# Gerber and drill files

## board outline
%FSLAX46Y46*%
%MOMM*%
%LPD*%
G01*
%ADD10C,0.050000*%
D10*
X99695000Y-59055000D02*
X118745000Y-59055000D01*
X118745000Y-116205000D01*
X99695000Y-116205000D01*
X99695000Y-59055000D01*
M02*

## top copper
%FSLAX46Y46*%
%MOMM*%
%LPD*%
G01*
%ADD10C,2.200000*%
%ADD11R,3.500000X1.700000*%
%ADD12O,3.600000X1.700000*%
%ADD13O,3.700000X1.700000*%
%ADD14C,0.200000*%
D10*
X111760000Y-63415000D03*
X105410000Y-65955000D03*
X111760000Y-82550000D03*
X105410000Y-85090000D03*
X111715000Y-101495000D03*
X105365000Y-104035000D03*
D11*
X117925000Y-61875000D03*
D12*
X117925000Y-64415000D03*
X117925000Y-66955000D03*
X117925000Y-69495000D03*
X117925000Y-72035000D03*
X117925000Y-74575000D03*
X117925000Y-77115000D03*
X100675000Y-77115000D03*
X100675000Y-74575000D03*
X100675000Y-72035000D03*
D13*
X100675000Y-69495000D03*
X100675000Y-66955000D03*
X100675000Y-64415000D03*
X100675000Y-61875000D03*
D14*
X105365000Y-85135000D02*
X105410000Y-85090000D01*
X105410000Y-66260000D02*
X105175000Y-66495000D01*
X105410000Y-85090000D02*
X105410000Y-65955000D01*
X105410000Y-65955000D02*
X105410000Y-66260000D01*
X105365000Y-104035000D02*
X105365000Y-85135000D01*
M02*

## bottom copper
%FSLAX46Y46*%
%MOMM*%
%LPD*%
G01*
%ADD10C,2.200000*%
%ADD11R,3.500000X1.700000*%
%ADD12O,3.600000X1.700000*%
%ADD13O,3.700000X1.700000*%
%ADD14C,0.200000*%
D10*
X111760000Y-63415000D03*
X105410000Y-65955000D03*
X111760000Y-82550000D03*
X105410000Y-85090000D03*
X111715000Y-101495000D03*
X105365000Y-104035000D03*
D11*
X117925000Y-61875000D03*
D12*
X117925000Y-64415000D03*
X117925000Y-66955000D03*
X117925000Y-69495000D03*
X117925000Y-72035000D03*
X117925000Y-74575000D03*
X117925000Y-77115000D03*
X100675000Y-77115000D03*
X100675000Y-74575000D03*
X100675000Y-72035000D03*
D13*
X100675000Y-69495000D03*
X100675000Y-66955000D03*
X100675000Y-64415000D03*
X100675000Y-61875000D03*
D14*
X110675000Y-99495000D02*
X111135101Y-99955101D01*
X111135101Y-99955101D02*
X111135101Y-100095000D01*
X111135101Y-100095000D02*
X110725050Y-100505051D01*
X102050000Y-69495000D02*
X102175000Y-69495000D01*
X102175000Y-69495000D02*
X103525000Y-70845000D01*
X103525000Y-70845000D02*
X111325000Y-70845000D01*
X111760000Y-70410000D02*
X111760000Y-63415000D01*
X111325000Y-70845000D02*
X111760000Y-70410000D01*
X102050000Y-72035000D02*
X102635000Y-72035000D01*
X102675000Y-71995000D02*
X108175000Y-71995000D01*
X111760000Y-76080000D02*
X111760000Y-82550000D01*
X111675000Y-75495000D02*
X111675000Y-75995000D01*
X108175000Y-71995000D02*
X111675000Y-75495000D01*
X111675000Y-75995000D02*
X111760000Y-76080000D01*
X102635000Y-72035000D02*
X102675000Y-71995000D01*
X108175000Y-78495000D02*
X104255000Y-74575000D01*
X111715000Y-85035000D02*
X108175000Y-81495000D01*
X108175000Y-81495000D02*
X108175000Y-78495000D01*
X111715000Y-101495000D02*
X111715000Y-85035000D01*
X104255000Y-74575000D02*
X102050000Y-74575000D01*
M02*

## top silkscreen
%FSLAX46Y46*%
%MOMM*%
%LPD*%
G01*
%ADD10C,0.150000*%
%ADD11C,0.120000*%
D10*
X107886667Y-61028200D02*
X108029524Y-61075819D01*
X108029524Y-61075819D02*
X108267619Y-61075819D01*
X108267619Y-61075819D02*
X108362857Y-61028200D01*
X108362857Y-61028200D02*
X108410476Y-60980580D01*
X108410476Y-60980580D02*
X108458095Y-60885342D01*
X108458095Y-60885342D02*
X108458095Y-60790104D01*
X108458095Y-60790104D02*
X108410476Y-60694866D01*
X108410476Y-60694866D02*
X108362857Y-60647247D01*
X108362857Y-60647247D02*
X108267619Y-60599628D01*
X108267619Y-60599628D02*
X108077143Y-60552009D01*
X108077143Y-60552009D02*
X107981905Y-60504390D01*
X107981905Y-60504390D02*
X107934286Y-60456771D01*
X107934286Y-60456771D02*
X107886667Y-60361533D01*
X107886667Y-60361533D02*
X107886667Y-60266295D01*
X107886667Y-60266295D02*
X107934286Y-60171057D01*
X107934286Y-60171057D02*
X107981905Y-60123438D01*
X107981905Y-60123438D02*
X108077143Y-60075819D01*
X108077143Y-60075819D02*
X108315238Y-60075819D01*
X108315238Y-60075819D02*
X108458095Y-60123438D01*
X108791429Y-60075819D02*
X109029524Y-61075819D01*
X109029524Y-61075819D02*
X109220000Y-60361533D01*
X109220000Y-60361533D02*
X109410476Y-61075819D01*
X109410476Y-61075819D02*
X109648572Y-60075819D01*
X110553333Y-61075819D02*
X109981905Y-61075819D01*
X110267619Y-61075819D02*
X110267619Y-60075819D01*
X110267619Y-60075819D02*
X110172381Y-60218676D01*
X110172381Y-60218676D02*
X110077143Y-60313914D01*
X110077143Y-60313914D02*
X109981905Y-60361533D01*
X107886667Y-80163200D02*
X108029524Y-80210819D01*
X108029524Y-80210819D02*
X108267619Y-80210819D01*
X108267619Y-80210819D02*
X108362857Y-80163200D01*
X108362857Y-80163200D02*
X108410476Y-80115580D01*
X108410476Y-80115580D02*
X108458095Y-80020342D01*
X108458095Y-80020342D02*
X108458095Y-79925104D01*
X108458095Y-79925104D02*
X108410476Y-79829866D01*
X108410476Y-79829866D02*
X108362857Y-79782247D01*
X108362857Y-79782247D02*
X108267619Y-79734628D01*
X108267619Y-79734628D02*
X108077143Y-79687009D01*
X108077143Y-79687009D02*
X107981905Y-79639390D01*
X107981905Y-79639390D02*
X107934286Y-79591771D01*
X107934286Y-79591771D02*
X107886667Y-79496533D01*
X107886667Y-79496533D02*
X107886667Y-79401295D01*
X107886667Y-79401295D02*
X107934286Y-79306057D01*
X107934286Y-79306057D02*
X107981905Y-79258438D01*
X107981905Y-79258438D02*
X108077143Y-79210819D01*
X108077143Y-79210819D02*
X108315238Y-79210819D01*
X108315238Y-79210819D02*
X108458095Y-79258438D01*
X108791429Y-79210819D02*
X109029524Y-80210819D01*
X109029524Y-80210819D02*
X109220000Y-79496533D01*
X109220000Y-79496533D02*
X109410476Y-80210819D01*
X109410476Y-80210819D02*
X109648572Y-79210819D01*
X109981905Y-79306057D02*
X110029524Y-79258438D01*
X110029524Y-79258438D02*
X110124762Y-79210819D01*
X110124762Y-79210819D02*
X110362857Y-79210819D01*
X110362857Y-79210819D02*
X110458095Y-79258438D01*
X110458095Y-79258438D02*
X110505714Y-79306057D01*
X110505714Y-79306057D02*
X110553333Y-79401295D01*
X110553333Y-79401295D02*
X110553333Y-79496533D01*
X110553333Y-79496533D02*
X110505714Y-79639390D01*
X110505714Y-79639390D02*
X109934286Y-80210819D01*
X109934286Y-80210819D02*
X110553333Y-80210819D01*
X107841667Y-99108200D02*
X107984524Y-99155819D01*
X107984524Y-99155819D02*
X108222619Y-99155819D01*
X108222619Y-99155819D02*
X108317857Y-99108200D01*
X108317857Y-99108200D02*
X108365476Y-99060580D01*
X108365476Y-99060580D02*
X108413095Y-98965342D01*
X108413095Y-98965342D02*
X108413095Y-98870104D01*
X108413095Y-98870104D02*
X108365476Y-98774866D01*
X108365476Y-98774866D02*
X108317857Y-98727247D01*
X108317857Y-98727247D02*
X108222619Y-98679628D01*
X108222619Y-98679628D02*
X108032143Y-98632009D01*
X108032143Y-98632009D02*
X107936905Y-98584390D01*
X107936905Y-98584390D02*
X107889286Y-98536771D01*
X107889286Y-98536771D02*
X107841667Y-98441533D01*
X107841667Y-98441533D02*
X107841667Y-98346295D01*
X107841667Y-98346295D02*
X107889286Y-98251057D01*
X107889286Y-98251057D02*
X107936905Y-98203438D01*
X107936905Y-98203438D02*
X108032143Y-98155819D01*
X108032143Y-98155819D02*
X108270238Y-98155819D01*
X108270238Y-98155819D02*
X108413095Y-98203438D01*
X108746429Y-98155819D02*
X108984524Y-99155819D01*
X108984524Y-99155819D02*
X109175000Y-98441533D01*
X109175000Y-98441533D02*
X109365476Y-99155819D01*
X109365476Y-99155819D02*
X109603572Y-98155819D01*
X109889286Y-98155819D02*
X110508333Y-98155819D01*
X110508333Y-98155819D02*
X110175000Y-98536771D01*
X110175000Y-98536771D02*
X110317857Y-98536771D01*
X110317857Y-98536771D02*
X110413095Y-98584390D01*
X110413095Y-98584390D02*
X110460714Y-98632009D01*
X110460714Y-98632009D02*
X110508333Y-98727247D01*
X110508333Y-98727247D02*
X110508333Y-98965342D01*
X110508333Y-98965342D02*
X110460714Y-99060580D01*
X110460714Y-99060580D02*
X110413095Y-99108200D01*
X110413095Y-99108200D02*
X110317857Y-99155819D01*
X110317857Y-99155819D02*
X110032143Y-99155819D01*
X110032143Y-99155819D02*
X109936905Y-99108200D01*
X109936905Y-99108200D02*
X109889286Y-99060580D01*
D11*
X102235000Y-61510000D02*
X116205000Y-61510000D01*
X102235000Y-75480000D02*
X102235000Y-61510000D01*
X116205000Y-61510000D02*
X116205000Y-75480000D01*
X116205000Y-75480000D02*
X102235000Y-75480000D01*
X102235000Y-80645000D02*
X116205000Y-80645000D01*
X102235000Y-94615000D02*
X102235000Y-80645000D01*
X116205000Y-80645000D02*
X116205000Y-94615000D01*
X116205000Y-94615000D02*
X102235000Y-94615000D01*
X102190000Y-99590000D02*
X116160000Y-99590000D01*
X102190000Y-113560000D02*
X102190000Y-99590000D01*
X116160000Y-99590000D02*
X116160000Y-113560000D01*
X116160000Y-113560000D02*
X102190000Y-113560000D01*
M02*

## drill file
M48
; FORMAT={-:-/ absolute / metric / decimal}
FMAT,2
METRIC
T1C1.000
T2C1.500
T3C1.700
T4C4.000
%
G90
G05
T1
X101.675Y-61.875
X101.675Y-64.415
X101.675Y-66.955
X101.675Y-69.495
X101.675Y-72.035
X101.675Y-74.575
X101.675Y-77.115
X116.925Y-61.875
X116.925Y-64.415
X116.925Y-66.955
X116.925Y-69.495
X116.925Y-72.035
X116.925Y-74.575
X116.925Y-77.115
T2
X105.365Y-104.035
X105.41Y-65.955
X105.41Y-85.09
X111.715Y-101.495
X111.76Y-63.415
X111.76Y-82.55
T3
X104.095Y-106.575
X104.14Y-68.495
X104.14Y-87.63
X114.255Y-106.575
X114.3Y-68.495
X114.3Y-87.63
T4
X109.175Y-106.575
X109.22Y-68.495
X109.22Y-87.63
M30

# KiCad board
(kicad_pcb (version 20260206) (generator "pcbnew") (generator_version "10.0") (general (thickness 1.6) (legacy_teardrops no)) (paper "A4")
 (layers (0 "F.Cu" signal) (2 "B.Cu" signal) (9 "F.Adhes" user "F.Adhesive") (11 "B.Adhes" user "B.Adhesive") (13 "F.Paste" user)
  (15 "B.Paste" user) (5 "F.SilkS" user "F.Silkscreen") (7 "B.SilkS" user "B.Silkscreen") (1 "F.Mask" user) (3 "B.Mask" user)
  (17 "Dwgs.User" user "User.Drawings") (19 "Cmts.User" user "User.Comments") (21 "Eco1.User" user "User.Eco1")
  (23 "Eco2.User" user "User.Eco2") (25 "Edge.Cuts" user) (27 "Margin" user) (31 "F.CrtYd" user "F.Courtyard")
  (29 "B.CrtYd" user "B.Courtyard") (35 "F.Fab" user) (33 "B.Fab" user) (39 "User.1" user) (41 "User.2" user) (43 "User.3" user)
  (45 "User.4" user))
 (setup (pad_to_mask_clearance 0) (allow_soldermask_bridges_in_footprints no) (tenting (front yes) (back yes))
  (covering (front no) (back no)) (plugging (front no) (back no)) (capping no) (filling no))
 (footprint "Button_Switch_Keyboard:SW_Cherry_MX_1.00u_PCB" (layer "F.Cu") (at 111.76 63.415)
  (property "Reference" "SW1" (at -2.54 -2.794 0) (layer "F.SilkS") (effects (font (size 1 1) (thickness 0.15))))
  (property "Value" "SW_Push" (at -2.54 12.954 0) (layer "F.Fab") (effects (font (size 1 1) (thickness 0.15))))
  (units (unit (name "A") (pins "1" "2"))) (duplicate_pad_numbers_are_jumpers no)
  (fp_line (start -9.525 -1.905) (end 4.445 -1.905) (stroke (width 0.12) (type solid)) (layer "F.SilkS"))
  (fp_line (start -9.525 12.065) (end -9.525 -1.905) (stroke (width 0.12) (type solid)) (layer "F.SilkS"))
  (fp_line (start 4.445 -1.905) (end 4.445 12.065) (stroke (width 0.12) (type solid)) (layer "F.SilkS"))
  (fp_line (start 4.445 12.065) (end -9.525 12.065) (stroke (width 0.12) (type solid)) (layer "F.SilkS"))
  (pad "" np_thru_hole circle (at -7.62 5.08) (size 1.7 1.7) (drill 1.7) (layers "*.Cu" "*.Mask"))
  (pad "" np_thru_hole circle (at -2.54 5.08) (size 4 4) (drill 4) (layers "*.Cu" "*.Mask"))
  (pad "" np_thru_hole circle (at 2.54 5.08) (size 1.7 1.7) (drill 1.7) (layers "*.Cu" "*.Mask"))
  (pad "1" thru_hole circle (at 0 0) (size 2.2 2.2) (drill 1.5) (layers "*.Cu" "*.Mask") (remove_unused_layers no)
   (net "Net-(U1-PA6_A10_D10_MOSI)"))
  (pad "2" thru_hole circle (at -6.35 2.54) (size 2.2 2.2) (drill 1.5) (layers "*.Cu" "*.Mask") (remove_unused_layers no) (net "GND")))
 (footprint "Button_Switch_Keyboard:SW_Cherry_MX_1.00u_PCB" (layer "F.Cu") (at 111.76 82.55)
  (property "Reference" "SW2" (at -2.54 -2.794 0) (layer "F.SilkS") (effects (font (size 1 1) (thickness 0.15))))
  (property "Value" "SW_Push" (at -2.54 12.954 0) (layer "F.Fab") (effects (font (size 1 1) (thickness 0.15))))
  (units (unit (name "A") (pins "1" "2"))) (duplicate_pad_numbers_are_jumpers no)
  (fp_line (start -9.525 -1.905) (end 4.445 -1.905) (stroke (width 0.12) (type solid)) (layer "F.SilkS"))
  (fp_line (start -9.525 12.065) (end -9.525 -1.905) (stroke (width 0.12) (type solid)) (layer "F.SilkS"))
  (fp_line (start 4.445 -1.905) (end 4.445 12.065) (stroke (width 0.12) (type solid)) (layer "F.SilkS"))
  (fp_line (start 4.445 12.065) (end -9.525 12.065) (stroke (width 0.12) (type solid)) (layer "F.SilkS"))
  (pad "" np_thru_hole circle (at -7.62 5.08) (size 1.7 1.7) (drill 1.7) (layers "*.Cu" "*.Mask"))
  (pad "" np_thru_hole circle (at -2.54 5.08) (size 4 4) (drill 4) (layers "*.Cu" "*.Mask"))
  (pad "" np_thru_hole circle (at 2.54 5.08) (size 1.7 1.7) (drill 1.7) (layers "*.Cu" "*.Mask"))
  (pad "1" thru_hole circle (at 0 0) (size 2.2 2.2) (drill 1.5) (layers "*.Cu" "*.Mask") (remove_unused_layers no)
   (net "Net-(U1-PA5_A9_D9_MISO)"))
  (pad "2" thru_hole circle (at -6.35 2.54) (size 2.2 2.2) (drill 1.5) (layers "*.Cu" "*.Mask") (remove_unused_layers no) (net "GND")))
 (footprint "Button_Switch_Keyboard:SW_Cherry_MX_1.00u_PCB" (layer "F.Cu") (at 111.715 101.495)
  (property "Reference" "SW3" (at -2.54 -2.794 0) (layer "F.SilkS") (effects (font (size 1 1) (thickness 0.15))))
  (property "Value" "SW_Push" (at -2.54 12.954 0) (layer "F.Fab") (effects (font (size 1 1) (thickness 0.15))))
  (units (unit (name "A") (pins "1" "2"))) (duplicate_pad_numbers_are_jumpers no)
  (fp_line (start -9.525 -1.905) (end 4.445 -1.905) (stroke (width 0.12) (type solid)) (layer "F.SilkS"))
  (fp_line (start -9.525 12.065) (end -9.525 -1.905) (stroke (width 0.12) (type solid)) (layer "F.SilkS"))
  (fp_line (start 4.445 -1.905) (end 4.445 12.065) (stroke (width 0.12) (type solid)) (layer "F.SilkS"))
  (fp_line (start 4.445 12.065) (end -9.525 12.065) (stroke (width 0.12) (type solid)) (layer "F.SilkS"))
  (pad "" np_thru_hole circle (at -7.62 5.08) (size 1.7 1.7) (drill 1.7) (layers "*.Cu" "*.Mask"))
  (pad "" np_thru_hole circle (at -2.54 5.08) (size 4 4) (drill 4) (layers "*.Cu" "*.Mask"))
  (pad "" np_thru_hole circle (at 2.54 5.08) (size 1.7 1.7) (drill 1.7) (layers "*.Cu" "*.Mask"))
  (pad "1" thru_hole circle (at 0 0) (size 2.2 2.2) (drill 1.5) (layers "*.Cu" "*.Mask") (remove_unused_layers no)
   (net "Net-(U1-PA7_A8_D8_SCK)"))
  (pad "2" thru_hole circle (at -6.35 2.54) (size 2.2 2.2) (drill 1.5) (layers "*.Cu" "*.Mask") (remove_unused_layers no) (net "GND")))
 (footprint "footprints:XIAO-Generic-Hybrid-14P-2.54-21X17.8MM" (layer "B.Cu") (at 109.3 69.495 180)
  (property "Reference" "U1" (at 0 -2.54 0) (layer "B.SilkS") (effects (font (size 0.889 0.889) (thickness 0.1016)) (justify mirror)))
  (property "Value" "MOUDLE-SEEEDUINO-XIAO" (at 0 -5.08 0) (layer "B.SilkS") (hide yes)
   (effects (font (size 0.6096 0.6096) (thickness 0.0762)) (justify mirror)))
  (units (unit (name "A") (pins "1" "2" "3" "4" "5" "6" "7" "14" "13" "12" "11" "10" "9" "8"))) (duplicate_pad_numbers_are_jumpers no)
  (pad "1" thru_hole rect (at -7.625 7.62 180) (size 3.5 1.7) (drill 1 (offset -1 0)) (layers "*.Cu" "*.Mask") (remove_unused_layers no)
   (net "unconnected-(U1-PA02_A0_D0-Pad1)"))
  (pad "2" thru_hole oval (at -7.625 5.08 180) (size 3.6 1.7) (drill 1 (offset -1 0)) (layers "*.Cu" "*.Mask") (remove_unused_layers no)
   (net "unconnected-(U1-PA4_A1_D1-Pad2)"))
  (pad "3" thru_hole oval (at -7.625 2.54 180) (size 3.6 1.7) (drill 1 (offset -1 0)) (layers "*.Cu" "*.Mask") (remove_unused_layers no)
   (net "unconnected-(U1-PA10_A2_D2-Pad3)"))
  (pad "4" thru_hole oval (at -7.625 0 180) (size 3.6 1.7) (drill 1 (offset -1 0)) (layers "*.Cu" "*.Mask") (remove_unused_layers no)
   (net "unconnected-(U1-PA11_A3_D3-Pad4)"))
  (pad "5" thru_hole oval (at -7.625 -2.54 180) (size 3.6 1.7) (drill 1 (offset -1 0)) (layers "*.Cu" "*.Mask") (remove_unused_layers no)
   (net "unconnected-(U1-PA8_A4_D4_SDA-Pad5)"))
  (pad "6" thru_hole oval (at -7.625 -5.08) (size 3.6 1.7) (drill 1 (offset 1 0)) (layers "*.Cu" "*.Mask") (remove_unused_layers no)
   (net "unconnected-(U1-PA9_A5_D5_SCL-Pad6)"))
  (pad "7" thru_hole oval (at -7.625 -7.62 180) (size 3.6 1.7) (drill 1 (offset -1 0)) (layers "*.Cu" "*.Mask") (remove_unused_layers no)
   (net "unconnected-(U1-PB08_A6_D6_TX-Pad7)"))
  (pad "8" thru_hole oval (at 7.625 -7.62 180) (size 3.6 1.7) (drill 1 (offset 1 0)) (layers "*.Cu" "*.Mask") (remove_unused_layers no)
   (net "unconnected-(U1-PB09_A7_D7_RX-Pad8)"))
  (pad "9" thru_hole oval (at 7.625 -5.08 180) (size 3.6 1.7) (drill 1 (offset 1 0)) (layers "*.Cu" "*.Mask") (remove_unused_layers no)
   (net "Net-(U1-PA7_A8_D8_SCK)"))
  (pad "10" thru_hole oval (at 7.625 -2.54 180) (size 3.6 1.7) (drill 1 (offset 1 0)) (layers "*.Cu" "*.Mask") (remove_unused_layers no)
   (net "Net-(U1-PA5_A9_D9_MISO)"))
  (pad "11" thru_hole oval (at 7.625 0 180) (size 3.7 1.7) (drill 1 (offset 1 0)) (layers "*.Cu" "*.Mask") (remove_unused_layers no)
   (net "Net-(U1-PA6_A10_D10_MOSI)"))
  (pad "12" thru_hole oval (at 7.625 2.54 180) (size 3.7 1.7) (drill 1 (offset 1 0)) (layers "*.Cu" "*.Mask") (remove_unused_layers no)
   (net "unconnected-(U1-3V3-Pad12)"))
  (pad "13" thru_hole oval (at 7.625 5.08 180) (size 3.7 1.7) (drill 1 (offset 1 0)) (layers "*.Cu" "*.Mask") (remove_unused_layers no)
   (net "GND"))
  (pad "14" thru_hole oval (at 7.625 7.62 180) (size 3.7 1.7) (drill 1 (offset 1 0)) (layers "*.Cu" "*.Mask") (remove_unused_layers no)
   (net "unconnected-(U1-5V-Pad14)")))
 (gr_rect (start 99.695 59.055) (end 118.745 116.205) (stroke (width 0.05) (type default)) (fill no) (layer "Edge.Cuts"))
 (segment (start 110.675 99.495) (end 111.135101 99.955101) (width 0.2) (layer "B.Cu") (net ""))
 (segment (start 111.135101 99.955101) (end 111.135101 100.095) (width 0.2) (layer "B.Cu") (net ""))
 (segment (start 111.135101 100.095) (end 110.72505 100.505051) (width 0.2) (layer "B.Cu") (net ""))
 (segment (start 102.05 69.495) (end 102.175 69.495) (width 0.2) (layer "B.Cu") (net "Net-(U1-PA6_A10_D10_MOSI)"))
 (segment (start 102.175 69.495) (end 103.525 70.845) (width 0.2) (layer "B.Cu") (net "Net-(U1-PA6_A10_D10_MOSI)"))
 (segment (start 103.525 70.845) (end 111.325 70.845) (width 0.2) (layer "B.Cu") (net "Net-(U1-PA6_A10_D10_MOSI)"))
 (segment (start 111.76 70.41) (end 111.76 63.415) (width 0.2) (layer "B.Cu") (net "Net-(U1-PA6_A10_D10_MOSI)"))
 (segment (start 111.325 70.845) (end 111.76 70.41) (width 0.2) (layer "B.Cu") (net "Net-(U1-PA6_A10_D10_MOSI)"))
 (segment (start 105.365 85.135) (end 105.41 85.09) (width 0.2) (layer "F.Cu") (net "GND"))
 (segment (start 105.41 66.26) (end 105.175 66.495) (width 0.2) (layer "F.Cu") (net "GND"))
 (segment (start 105.41 85.09) (end 105.41 65.955) (width 0.2) (layer "F.Cu") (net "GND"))
 (segment (start 105.41 65.955) (end 105.41 66.26) (width 0.2) (layer "F.Cu") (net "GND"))
 (segment (start 105.365 104.035) (end 105.365 85.135) (width 0.2) (layer "F.Cu") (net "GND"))
 (segment (start 102.05 72.035) (end 102.635 72.035) (width 0.2) (layer "B.Cu") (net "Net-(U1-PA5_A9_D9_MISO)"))
 (segment (start 102.675 71.995) (end 108.175 71.995) (width 0.2) (layer "B.Cu") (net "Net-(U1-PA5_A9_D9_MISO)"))
 (segment (start 111.76 76.08) (end 111.76 82.55) (width 0.2) (layer "B.Cu") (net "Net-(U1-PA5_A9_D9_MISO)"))
 (segment (start 111.675 75.495) (end 111.675 75.995) (width 0.2) (layer "B.Cu") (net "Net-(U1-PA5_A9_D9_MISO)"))
 (segment (start 108.175 71.995) (end 111.675 75.495) (width 0.2) (layer "B.Cu") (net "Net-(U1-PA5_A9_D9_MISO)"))
 (segment (start 111.675 75.995) (end 111.76 76.08) (width 0.2) (layer "B.Cu") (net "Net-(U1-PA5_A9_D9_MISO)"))
 (segment (start 102.635 72.035) (end 102.675 71.995) (width 0.2) (layer "B.Cu") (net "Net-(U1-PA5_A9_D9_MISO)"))
 (segment (start 108.175 78.495) (end 104.255 74.575) (width 0.2) (layer "B.Cu") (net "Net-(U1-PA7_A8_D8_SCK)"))
 (segment (start 111.715 85.035) (end 108.175 81.495) (width 0.2) (layer "B.Cu") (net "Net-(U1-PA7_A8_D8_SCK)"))
 (segment (start 108.175 81.495) (end 108.175 78.495) (width 0.2) (layer "B.Cu") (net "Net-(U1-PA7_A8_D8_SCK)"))
 (segment (start 111.715 101.495) (end 111.715 85.035) (width 0.2) (layer "B.Cu") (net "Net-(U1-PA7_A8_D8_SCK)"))
 (segment (start 104.255 74.575) (end 102.05 74.575) (width 0.2) (layer "B.Cu") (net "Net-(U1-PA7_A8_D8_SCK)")))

